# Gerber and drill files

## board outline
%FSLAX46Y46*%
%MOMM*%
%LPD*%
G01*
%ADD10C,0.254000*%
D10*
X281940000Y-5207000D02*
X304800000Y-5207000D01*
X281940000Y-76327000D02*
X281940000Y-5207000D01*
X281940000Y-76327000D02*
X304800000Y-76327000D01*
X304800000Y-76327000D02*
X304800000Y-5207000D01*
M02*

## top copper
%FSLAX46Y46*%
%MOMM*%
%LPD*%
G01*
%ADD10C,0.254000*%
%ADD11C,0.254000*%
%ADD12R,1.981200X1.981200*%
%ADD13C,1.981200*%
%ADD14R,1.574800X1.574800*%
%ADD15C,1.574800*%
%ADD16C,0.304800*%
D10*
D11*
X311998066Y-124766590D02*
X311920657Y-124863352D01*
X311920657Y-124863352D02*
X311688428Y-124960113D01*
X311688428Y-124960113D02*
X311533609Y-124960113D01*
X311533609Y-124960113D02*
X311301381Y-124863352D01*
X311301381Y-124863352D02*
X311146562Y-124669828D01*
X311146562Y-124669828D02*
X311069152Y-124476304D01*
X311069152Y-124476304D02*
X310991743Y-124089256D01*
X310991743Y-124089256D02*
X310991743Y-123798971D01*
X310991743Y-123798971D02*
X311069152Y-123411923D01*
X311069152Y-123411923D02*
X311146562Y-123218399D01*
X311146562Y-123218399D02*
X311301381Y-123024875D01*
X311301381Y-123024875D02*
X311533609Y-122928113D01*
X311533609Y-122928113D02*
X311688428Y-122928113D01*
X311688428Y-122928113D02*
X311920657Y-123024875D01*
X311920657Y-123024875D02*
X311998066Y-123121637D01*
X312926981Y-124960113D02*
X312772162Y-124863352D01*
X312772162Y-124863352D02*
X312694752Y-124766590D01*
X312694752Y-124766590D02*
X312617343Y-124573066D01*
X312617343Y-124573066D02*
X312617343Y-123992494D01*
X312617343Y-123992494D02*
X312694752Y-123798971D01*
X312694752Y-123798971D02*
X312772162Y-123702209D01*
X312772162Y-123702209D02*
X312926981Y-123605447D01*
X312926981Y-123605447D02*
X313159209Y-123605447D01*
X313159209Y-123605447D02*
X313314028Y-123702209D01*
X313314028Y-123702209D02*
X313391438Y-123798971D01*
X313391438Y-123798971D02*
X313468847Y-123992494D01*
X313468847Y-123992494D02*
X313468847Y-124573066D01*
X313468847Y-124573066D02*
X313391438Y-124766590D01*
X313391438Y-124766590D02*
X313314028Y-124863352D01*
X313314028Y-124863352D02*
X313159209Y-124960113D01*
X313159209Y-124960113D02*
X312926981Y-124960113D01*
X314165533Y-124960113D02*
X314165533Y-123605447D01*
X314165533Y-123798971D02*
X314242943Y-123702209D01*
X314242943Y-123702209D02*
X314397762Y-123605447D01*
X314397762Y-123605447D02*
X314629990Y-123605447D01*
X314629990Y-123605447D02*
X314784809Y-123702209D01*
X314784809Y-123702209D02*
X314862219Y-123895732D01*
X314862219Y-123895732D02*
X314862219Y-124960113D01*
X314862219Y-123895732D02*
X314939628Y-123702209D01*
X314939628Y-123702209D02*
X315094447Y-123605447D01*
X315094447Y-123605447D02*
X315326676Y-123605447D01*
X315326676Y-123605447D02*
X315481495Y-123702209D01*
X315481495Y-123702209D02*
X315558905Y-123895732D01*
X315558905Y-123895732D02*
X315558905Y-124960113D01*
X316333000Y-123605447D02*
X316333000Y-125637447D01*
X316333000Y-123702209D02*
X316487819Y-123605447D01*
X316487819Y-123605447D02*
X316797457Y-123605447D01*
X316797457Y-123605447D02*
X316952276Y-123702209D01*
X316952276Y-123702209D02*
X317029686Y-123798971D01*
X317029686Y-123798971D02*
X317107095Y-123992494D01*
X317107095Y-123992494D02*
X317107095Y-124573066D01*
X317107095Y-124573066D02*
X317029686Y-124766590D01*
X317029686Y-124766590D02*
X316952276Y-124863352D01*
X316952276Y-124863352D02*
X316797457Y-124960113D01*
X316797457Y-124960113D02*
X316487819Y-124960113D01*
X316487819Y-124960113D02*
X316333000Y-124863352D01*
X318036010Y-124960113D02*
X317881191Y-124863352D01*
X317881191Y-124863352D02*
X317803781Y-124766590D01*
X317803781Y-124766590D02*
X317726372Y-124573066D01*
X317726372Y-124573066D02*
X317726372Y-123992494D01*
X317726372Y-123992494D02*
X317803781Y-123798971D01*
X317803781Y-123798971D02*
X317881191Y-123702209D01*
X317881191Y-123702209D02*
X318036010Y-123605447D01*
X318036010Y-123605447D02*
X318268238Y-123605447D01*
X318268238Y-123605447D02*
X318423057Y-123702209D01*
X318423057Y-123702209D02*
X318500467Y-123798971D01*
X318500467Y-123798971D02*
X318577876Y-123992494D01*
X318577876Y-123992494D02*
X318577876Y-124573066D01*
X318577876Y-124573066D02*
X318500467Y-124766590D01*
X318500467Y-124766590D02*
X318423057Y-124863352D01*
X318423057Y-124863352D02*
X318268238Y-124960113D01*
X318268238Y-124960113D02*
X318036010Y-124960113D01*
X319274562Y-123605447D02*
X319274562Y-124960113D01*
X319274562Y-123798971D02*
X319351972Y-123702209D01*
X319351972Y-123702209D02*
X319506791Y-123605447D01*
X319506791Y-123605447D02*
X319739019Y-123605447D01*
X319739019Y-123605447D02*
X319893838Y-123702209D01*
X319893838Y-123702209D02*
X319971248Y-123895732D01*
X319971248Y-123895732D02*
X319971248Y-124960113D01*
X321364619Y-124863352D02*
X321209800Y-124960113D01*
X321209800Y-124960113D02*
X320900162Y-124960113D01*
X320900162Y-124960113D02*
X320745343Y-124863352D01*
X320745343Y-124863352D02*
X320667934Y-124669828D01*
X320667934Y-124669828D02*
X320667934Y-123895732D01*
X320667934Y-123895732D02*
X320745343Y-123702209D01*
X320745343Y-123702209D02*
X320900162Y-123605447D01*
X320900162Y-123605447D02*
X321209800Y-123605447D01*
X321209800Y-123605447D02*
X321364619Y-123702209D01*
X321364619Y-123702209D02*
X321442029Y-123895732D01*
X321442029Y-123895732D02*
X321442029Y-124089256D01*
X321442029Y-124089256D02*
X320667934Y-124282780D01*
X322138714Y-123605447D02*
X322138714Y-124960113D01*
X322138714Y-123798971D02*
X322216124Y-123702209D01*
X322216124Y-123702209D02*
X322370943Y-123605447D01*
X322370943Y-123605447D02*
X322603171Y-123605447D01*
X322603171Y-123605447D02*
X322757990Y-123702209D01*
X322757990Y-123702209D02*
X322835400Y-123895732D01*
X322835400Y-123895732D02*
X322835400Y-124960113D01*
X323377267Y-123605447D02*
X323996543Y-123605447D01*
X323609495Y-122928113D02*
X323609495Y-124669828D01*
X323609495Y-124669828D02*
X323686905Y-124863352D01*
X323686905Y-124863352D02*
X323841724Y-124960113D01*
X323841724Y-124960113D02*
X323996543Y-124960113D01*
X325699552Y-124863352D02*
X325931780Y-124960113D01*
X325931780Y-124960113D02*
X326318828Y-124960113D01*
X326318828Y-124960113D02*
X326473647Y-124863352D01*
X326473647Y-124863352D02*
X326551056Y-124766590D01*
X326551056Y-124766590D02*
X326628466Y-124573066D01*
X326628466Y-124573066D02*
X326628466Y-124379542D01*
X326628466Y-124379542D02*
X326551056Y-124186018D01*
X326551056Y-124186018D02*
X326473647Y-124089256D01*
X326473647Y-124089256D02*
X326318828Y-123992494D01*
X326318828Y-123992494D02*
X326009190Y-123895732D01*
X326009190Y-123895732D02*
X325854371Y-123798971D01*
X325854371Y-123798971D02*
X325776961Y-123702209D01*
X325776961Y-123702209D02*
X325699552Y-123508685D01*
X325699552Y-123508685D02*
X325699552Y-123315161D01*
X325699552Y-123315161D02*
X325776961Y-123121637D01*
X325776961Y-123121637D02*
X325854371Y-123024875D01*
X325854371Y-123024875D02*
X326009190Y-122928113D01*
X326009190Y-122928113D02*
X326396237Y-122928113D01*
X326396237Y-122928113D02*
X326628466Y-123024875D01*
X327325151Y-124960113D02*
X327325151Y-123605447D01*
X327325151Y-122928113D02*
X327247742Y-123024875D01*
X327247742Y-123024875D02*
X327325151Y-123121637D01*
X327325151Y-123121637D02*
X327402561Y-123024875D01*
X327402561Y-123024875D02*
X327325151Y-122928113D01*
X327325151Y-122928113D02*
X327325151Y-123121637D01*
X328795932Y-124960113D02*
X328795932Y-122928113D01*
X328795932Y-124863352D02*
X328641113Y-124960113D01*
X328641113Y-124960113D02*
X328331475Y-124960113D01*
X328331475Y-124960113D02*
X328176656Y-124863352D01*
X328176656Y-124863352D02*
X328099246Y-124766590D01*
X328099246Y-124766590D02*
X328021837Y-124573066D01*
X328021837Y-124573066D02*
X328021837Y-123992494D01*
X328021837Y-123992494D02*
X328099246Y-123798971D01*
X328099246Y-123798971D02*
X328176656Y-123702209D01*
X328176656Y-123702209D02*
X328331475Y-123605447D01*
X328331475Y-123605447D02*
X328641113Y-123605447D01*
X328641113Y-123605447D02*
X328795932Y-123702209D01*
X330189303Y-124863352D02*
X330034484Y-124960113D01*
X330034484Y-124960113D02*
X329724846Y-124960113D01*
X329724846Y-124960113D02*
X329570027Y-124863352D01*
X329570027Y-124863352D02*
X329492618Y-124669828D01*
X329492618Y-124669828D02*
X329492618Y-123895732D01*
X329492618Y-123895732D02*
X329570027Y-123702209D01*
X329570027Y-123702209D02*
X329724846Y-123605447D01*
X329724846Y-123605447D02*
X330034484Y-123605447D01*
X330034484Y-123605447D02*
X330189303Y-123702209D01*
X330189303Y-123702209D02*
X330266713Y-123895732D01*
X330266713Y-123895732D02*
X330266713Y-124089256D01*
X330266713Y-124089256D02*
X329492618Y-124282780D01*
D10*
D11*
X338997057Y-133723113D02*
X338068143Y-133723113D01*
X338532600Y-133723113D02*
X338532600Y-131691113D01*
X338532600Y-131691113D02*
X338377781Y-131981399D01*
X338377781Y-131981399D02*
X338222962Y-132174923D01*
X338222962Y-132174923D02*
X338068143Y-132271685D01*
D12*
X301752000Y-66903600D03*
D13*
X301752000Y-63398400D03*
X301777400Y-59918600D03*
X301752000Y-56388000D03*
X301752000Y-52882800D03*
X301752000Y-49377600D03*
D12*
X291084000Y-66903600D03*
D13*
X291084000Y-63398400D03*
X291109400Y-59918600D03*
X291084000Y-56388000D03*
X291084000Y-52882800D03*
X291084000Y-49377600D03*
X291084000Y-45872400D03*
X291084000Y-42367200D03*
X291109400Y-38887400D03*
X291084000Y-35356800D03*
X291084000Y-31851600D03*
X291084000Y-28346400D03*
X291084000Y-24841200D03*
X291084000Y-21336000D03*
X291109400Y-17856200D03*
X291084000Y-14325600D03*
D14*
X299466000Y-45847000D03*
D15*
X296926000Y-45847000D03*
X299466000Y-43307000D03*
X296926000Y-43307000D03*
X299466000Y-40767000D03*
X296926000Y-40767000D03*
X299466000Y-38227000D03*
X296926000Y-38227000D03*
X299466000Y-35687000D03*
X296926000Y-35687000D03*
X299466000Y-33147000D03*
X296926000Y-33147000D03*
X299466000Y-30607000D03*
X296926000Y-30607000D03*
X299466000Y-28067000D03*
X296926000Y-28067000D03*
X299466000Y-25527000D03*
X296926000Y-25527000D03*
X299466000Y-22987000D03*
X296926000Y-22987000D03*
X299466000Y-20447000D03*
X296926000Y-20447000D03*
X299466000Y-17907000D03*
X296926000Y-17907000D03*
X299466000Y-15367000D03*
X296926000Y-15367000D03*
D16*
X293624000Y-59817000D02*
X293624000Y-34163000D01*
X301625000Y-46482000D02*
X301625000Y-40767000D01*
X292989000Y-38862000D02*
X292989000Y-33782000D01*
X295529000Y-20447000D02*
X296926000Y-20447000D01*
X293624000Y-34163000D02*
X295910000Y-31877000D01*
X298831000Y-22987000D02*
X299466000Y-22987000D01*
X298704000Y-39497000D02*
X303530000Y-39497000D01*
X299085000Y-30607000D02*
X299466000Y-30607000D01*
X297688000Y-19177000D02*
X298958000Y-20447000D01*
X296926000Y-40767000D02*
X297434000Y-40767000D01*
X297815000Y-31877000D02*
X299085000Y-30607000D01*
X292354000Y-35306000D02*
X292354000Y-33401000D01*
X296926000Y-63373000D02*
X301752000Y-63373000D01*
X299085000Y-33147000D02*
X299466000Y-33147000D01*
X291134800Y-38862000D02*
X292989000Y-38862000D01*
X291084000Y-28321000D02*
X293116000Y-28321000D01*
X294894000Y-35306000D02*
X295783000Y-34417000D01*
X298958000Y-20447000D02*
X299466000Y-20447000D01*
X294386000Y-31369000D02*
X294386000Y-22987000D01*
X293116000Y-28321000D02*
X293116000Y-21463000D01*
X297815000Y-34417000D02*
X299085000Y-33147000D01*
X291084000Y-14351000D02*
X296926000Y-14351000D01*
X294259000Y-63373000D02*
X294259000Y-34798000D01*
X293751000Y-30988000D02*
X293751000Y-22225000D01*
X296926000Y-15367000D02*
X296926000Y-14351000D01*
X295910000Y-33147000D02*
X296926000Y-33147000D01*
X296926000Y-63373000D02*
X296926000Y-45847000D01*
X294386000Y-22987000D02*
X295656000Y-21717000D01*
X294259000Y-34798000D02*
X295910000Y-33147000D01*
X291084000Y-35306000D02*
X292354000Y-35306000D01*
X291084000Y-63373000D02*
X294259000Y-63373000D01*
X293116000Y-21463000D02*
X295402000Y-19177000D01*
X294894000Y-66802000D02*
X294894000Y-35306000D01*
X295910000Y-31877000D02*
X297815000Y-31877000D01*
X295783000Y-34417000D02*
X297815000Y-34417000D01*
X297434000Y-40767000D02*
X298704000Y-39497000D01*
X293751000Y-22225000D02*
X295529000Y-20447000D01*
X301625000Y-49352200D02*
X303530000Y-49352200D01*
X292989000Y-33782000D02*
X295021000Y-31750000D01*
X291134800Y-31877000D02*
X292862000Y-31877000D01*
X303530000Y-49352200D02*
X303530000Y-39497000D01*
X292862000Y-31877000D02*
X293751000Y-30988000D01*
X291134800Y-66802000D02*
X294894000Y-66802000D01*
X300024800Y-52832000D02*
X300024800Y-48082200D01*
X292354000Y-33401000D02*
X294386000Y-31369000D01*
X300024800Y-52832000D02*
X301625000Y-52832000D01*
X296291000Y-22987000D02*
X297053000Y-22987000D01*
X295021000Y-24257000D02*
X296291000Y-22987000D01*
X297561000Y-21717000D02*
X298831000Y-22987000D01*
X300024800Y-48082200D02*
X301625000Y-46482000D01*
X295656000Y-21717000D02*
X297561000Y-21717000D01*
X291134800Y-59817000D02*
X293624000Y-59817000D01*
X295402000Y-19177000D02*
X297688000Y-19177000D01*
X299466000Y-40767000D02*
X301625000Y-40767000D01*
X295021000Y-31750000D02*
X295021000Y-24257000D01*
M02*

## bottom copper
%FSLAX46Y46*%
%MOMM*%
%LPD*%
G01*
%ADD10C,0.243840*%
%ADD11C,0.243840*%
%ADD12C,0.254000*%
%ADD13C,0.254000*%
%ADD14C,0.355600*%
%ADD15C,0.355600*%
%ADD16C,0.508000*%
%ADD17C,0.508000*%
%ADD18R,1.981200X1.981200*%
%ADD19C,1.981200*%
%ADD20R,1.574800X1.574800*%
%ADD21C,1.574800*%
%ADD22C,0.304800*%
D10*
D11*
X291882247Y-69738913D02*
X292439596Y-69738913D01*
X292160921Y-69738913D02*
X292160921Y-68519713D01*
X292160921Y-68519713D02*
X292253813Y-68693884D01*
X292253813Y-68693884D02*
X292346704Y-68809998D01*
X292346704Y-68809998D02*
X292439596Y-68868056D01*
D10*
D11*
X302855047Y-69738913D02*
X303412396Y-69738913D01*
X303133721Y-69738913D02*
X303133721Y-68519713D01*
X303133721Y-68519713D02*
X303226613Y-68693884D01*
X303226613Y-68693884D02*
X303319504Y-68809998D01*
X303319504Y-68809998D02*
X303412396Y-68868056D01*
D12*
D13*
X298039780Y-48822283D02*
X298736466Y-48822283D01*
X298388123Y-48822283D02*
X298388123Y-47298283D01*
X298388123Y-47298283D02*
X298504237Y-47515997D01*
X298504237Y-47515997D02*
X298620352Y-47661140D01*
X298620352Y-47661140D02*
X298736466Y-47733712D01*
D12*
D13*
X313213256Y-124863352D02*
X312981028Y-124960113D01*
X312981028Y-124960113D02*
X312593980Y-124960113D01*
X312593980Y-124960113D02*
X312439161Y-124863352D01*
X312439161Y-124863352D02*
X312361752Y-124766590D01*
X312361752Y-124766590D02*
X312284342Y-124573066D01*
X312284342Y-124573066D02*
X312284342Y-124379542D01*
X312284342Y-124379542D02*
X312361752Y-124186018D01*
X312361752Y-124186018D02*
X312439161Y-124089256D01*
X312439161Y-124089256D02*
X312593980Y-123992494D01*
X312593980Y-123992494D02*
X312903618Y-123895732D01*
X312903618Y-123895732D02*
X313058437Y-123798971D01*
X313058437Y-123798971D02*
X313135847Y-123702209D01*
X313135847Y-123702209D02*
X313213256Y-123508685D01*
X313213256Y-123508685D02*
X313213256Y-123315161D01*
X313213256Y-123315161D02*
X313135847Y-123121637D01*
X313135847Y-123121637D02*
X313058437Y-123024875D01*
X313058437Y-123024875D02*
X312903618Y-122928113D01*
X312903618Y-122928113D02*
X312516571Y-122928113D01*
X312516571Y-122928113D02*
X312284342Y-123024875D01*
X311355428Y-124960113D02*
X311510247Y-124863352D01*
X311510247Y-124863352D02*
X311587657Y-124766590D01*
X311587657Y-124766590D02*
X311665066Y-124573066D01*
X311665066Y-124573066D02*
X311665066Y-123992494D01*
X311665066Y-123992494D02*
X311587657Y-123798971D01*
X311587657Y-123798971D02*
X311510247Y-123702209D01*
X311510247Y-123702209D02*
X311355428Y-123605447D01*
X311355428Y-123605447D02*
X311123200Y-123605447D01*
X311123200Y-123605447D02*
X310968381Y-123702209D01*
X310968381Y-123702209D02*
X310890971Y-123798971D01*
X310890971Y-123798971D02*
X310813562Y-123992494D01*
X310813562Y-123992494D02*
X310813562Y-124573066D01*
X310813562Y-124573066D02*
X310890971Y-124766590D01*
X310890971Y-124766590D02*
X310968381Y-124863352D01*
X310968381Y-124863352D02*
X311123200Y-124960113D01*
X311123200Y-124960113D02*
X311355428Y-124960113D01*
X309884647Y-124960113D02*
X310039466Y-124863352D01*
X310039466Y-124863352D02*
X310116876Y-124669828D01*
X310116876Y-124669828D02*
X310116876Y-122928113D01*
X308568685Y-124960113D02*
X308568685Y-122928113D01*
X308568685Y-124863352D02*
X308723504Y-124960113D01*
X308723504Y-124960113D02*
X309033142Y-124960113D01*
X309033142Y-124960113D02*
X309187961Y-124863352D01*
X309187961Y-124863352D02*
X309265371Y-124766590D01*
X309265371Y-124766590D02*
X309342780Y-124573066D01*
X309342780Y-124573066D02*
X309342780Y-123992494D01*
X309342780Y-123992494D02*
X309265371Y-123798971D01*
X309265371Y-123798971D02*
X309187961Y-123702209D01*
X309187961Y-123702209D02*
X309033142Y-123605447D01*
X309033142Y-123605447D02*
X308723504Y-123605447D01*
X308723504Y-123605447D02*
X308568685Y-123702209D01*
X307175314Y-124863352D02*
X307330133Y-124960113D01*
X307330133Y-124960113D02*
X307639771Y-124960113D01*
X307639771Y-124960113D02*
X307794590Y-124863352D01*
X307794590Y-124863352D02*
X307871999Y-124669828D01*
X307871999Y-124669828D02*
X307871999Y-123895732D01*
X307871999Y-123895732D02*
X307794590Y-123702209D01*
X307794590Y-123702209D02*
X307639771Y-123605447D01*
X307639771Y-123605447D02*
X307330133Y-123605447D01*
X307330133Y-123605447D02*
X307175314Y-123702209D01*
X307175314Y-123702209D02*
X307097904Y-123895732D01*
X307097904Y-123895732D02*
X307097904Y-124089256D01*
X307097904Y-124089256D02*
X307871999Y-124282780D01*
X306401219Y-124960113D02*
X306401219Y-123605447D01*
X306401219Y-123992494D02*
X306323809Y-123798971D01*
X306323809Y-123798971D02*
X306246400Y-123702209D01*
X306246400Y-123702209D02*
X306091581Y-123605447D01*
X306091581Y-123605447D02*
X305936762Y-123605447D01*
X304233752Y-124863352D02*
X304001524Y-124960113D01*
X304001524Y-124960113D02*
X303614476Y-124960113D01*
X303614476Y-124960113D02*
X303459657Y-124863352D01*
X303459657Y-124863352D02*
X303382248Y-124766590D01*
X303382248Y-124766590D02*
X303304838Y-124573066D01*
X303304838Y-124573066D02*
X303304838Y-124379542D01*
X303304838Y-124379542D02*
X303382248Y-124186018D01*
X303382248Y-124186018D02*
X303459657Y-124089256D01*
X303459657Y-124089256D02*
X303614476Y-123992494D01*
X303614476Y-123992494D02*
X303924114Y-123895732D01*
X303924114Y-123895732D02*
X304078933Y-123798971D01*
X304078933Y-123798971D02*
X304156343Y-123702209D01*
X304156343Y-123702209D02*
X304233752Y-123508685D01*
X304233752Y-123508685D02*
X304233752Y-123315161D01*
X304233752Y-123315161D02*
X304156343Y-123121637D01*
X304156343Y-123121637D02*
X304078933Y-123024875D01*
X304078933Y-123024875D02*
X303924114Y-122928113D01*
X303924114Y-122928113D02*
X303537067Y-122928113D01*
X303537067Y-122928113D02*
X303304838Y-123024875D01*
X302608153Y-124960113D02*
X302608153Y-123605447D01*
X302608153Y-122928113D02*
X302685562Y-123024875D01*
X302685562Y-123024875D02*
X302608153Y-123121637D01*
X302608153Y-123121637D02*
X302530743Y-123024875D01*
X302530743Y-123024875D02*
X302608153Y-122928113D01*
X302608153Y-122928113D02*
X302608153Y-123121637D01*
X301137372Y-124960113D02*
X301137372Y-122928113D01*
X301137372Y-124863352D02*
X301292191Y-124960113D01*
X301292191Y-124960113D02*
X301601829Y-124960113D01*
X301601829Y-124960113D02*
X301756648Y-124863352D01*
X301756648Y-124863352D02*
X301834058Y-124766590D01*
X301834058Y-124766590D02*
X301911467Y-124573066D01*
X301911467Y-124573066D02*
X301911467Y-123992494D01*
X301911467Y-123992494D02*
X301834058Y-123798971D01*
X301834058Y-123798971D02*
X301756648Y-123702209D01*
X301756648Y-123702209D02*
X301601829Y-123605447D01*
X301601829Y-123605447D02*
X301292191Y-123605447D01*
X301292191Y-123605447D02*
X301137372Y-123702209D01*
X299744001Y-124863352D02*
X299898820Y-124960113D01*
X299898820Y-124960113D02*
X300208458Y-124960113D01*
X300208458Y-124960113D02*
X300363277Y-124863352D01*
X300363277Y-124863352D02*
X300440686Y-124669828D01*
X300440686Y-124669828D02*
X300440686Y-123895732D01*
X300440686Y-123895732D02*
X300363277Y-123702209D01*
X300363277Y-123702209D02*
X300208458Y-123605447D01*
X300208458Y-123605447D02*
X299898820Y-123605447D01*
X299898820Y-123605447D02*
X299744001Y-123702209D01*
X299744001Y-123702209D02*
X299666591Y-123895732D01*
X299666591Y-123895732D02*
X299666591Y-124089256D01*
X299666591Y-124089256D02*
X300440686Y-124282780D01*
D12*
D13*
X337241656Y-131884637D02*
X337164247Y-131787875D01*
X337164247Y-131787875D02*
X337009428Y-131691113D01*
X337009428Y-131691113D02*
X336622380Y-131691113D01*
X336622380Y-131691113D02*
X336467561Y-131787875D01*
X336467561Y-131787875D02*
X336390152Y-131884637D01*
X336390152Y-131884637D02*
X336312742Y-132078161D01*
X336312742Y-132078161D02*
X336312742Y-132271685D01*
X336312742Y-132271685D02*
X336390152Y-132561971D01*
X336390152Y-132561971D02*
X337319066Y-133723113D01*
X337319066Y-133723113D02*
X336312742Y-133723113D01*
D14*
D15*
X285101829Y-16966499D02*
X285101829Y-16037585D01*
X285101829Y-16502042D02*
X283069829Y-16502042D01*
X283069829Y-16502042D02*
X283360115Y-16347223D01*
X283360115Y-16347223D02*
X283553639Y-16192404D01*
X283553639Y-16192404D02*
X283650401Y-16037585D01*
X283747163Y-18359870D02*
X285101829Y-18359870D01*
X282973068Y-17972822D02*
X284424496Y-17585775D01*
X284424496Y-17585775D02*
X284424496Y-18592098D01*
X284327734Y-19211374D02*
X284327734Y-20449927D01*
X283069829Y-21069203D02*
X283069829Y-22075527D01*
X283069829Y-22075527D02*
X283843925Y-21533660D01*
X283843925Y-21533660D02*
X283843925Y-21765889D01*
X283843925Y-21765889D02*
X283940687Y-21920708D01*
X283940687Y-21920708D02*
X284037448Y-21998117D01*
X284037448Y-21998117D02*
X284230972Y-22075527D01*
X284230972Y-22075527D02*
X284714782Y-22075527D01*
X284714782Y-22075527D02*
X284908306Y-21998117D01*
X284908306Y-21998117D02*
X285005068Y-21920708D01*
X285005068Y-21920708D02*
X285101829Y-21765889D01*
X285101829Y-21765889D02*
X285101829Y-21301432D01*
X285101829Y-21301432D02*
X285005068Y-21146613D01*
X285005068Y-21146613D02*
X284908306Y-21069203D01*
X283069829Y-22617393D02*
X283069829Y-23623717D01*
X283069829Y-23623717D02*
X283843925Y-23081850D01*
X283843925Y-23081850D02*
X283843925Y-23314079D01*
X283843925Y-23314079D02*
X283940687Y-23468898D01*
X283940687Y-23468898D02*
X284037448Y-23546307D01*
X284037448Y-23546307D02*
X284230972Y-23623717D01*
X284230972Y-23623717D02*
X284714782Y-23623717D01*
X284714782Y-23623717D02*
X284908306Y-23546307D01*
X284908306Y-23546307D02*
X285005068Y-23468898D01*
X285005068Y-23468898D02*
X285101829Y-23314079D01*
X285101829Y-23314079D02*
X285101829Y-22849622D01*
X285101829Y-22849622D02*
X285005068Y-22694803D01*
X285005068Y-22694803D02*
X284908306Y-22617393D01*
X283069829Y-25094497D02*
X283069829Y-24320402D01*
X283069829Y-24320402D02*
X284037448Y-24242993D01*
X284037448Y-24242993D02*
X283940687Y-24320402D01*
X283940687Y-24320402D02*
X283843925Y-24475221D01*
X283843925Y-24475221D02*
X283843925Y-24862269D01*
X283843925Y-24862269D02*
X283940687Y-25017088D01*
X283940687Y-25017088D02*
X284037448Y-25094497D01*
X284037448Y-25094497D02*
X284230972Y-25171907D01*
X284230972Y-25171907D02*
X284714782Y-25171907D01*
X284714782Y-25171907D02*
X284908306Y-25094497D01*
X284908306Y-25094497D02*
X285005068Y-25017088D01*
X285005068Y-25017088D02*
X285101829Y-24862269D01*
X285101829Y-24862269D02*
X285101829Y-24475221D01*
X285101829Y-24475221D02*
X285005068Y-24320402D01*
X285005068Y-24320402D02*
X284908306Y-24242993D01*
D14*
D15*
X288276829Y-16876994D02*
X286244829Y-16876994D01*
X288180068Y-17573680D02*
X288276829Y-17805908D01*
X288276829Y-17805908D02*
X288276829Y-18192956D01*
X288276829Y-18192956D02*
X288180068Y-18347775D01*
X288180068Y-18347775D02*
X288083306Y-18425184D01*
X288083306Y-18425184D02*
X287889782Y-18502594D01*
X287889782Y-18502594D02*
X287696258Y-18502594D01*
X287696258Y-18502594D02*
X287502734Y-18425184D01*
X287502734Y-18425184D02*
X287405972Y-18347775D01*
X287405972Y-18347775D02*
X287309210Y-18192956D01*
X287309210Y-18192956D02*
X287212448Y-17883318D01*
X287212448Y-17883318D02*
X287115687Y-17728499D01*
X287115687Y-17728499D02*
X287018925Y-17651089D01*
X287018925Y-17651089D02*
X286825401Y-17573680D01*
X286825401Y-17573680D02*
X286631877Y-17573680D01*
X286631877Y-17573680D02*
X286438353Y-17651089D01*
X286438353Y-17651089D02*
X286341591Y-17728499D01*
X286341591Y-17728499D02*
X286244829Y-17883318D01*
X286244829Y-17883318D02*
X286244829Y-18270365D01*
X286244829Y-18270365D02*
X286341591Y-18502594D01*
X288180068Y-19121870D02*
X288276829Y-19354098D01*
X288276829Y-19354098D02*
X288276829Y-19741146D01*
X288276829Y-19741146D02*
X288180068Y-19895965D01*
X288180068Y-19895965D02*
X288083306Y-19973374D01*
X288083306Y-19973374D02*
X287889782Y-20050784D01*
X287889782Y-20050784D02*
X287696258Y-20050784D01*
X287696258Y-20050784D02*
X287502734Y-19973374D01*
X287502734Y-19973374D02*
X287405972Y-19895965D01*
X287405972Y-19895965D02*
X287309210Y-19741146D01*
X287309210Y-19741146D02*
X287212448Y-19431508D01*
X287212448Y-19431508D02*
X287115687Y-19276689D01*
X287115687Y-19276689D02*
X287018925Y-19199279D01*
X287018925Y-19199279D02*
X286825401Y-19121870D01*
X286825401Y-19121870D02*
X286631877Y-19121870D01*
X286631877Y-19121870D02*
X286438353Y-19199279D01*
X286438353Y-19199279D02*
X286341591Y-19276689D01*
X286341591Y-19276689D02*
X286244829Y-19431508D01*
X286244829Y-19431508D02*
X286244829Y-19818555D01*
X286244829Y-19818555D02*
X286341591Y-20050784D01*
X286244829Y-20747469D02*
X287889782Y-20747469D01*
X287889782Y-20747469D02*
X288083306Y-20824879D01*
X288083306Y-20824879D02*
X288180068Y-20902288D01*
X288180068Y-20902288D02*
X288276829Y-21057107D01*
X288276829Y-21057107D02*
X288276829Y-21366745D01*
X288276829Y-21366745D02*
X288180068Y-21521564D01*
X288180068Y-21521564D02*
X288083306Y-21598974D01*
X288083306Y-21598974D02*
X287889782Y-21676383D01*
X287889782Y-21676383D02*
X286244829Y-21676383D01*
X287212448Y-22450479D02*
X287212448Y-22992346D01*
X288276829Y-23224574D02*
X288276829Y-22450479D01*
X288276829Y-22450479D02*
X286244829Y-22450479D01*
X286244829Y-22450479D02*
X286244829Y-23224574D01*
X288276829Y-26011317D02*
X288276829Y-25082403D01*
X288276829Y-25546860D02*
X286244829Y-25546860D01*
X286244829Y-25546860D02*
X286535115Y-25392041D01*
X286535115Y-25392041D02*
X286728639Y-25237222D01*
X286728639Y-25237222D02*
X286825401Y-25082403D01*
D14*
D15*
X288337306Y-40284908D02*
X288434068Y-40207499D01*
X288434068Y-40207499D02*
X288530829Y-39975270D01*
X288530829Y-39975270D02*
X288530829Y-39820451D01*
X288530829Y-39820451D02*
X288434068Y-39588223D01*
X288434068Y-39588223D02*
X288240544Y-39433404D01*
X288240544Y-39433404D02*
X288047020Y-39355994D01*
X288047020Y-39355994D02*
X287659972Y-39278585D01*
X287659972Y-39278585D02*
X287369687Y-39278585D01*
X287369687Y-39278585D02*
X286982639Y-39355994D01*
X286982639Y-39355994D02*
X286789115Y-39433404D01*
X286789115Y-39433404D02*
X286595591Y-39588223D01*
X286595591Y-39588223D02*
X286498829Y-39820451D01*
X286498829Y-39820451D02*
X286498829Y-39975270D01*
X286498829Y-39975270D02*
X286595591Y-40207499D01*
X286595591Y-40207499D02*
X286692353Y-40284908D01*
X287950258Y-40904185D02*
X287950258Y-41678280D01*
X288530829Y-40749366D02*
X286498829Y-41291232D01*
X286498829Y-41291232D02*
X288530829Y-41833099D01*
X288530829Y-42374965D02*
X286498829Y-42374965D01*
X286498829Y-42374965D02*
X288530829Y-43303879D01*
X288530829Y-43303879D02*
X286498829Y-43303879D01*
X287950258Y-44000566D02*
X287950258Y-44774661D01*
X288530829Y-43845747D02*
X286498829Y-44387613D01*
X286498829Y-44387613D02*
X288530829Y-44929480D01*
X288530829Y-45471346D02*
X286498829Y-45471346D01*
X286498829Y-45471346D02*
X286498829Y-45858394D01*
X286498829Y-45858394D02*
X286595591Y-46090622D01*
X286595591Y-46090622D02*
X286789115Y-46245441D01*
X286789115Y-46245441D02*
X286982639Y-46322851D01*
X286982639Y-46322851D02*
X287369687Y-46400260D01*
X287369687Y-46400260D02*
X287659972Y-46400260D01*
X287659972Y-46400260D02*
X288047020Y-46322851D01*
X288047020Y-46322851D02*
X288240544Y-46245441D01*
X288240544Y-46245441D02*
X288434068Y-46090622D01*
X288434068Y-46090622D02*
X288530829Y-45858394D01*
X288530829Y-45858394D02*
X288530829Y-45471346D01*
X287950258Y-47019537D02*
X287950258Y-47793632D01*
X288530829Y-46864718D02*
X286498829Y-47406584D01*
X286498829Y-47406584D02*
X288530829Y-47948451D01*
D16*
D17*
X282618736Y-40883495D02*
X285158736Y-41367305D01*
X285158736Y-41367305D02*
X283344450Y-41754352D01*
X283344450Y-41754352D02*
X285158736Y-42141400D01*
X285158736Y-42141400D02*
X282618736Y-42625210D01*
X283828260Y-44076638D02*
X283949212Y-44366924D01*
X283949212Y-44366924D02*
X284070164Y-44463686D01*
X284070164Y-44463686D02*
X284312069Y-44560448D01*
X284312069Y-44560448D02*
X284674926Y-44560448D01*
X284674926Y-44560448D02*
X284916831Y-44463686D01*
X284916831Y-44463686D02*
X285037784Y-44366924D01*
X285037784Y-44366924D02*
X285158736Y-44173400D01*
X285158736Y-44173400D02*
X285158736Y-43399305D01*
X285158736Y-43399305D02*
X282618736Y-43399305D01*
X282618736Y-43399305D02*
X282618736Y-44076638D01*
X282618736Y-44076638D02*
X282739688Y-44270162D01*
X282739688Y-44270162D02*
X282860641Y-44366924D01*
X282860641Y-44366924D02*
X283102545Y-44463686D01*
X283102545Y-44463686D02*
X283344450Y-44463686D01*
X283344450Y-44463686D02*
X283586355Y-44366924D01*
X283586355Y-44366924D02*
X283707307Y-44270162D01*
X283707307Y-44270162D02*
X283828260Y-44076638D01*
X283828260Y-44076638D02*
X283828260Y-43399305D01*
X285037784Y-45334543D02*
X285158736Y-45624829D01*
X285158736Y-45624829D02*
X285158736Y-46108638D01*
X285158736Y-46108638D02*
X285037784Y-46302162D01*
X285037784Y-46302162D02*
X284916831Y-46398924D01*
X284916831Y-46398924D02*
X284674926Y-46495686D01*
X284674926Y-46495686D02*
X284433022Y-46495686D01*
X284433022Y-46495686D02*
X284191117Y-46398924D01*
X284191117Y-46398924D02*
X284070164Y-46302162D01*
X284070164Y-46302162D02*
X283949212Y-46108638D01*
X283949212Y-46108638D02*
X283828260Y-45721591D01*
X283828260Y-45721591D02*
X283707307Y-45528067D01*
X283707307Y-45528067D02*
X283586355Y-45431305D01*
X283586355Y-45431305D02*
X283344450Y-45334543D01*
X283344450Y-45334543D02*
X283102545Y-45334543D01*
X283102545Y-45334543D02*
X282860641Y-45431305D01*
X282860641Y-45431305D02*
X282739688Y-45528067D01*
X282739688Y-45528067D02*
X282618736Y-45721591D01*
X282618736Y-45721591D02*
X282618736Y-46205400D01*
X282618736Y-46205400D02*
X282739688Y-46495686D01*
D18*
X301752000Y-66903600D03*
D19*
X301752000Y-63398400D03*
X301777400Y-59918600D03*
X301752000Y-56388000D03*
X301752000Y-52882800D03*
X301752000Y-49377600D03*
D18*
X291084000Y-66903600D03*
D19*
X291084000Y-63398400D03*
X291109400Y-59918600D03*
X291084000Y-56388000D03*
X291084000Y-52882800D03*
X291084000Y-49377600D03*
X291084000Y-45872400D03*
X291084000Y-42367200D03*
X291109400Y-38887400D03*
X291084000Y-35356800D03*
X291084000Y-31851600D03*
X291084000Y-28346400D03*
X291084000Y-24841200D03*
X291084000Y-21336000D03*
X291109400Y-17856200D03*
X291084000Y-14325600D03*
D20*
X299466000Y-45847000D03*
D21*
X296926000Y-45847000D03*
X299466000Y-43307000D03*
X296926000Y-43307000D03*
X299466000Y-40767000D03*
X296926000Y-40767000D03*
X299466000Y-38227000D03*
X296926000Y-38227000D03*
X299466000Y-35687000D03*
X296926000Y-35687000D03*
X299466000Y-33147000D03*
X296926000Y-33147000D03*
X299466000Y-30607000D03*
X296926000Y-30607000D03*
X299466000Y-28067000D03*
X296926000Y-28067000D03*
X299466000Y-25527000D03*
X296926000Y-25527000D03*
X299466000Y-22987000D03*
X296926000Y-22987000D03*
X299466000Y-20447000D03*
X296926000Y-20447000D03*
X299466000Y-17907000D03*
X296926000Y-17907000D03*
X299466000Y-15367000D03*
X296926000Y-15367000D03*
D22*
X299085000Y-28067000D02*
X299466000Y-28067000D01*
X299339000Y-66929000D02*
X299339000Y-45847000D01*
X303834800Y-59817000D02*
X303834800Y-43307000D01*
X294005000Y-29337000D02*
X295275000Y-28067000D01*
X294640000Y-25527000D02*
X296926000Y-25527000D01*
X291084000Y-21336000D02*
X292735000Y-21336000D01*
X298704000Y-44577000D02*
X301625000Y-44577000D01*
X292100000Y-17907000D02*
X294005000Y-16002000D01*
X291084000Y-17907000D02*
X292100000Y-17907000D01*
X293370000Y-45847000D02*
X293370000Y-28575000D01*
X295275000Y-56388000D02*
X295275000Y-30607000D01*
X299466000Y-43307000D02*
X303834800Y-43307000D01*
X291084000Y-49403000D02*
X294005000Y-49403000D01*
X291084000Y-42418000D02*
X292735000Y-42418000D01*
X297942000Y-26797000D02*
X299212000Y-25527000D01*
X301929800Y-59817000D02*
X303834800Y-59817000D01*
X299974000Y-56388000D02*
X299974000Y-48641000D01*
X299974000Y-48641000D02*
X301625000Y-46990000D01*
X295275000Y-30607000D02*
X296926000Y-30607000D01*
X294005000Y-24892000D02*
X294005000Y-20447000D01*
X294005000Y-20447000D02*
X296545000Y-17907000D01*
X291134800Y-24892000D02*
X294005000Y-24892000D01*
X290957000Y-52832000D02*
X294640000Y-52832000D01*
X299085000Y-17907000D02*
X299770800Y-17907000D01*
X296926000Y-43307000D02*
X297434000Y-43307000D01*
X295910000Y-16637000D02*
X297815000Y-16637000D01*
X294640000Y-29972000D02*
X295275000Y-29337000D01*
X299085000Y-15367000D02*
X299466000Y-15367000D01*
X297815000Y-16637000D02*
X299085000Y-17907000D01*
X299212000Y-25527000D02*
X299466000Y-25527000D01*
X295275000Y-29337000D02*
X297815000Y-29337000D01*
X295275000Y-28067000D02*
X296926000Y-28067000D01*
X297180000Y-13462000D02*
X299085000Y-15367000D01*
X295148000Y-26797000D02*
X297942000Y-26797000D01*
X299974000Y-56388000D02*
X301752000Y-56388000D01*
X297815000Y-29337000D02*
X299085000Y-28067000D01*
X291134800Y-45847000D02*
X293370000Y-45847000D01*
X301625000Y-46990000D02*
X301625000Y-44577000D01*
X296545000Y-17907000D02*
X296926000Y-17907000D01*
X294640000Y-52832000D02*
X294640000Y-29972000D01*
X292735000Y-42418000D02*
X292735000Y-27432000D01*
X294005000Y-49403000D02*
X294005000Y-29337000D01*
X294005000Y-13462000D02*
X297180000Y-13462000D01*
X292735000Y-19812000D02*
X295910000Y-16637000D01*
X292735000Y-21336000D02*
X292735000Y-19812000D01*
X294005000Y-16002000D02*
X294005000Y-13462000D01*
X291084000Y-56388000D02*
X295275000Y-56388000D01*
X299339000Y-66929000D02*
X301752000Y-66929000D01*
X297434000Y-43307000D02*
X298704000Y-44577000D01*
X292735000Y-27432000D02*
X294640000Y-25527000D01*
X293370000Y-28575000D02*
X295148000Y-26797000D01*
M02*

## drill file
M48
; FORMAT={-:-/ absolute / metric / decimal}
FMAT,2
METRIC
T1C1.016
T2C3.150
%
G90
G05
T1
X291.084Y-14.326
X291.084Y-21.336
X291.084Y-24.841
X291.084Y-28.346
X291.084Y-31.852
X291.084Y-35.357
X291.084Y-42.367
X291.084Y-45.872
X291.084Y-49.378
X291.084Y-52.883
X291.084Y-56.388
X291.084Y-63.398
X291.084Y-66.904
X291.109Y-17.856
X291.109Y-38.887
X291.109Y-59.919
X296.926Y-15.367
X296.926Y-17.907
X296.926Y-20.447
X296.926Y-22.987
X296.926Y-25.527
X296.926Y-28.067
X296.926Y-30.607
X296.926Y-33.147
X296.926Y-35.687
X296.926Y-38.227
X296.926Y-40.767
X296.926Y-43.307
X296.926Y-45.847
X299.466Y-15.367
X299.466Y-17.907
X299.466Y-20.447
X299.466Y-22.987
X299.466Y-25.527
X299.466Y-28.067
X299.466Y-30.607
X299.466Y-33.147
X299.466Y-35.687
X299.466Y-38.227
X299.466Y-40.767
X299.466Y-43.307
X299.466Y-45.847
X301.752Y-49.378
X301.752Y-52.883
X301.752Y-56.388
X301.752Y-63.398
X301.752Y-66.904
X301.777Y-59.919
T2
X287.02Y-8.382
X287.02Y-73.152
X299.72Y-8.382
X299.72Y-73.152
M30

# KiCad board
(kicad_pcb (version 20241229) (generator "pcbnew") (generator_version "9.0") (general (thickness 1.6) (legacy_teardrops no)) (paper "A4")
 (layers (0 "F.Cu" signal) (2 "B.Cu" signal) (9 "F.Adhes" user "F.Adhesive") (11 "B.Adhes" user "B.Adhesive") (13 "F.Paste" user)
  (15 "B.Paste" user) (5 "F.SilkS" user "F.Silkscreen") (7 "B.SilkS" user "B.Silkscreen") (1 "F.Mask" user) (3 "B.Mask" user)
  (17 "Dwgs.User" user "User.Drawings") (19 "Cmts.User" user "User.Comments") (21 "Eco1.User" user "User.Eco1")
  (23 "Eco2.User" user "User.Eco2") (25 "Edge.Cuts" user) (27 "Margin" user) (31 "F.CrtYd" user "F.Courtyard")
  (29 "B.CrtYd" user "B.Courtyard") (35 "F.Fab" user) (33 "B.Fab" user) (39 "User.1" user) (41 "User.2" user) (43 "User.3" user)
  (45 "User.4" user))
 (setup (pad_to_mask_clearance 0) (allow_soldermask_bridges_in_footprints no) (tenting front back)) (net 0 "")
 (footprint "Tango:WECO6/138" (layer "F.Cu") (at 301.752 66.9036)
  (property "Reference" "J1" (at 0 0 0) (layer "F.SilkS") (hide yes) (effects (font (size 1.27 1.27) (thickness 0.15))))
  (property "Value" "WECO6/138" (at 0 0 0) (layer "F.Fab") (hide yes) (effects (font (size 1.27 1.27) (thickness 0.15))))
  (pad "1" thru_hole rect (at 0 0) (size 1.9812 1.9812) (drill 1.016) (layers "*.Cu" "*.Mask") (remove_unused_layers no)
   (thermal_bridge_angle 45))
  (pad "2" thru_hole circle (at 0 -3.5052) (size 1.9812 1.9812) (drill 1.016) (layers "*.Cu" "*.Mask") (remove_unused_layers no))
  (pad "3" thru_hole circle (at 0.0254 -6.985) (size 1.9812 1.9812) (drill 1.016) (layers "*.Cu" "*.Mask") (remove_unused_layers no))
  (pad "4" thru_hole circle (at 0 -10.5156) (size 1.9812 1.9812) (drill 1.016) (layers "*.Cu" "*.Mask") (remove_unused_layers no))
  (pad "5" thru_hole circle (at 0 -14.0208) (size 1.9812 1.9812) (drill 1.016) (layers "*.Cu" "*.Mask") (remove_unused_layers no))
  (pad "6" thru_hole circle (at 0 -17.526) (size 1.9812 1.9812) (drill 1.016) (layers "*.Cu" "*.Mask") (remove_unused_layers no)))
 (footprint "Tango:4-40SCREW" (layer "F.Cu") (at 299.72 73.152)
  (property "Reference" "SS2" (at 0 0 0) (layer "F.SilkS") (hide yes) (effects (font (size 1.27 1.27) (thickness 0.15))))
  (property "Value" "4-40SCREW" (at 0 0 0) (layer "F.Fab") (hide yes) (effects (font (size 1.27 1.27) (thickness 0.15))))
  (pad "" np_thru_hole circle (at 0 0) (size 3.1496 3.1496) (drill 3.1496) (layers "*.Cu" "*.Mask")))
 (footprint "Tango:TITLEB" (layer "F.Cu") (at 358.14 139.827)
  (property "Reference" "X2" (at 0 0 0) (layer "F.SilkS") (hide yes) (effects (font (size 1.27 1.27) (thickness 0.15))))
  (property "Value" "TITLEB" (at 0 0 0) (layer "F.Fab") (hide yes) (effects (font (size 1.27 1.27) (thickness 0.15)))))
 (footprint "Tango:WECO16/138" (layer "F.Cu") (at 291.084 66.9036)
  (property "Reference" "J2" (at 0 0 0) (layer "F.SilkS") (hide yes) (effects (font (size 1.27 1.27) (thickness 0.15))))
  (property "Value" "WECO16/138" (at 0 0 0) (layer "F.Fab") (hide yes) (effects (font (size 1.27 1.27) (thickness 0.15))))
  (pad "1" thru_hole rect (at 0 0) (size 1.9812 1.9812) (drill 1.016) (layers "*.Cu" "*.Mask") (remove_unused_layers no)
   (thermal_bridge_angle 45))
  (pad "2" thru_hole circle (at 0 -3.5052) (size 1.9812 1.9812) (drill 1.016) (layers "*.Cu" "*.Mask") (remove_unused_layers no))
  (pad "3" thru_hole circle (at 0.0254 -6.985) (size 1.9812 1.9812) (drill 1.016) (layers "*.Cu" "*.Mask") (remove_unused_layers no))
  (pad "4" thru_hole circle (at 0 -10.5156) (size 1.9812 1.9812) (drill 1.016) (layers "*.Cu" "*.Mask") (remove_unused_layers no))
  (pad "5" thru_hole circle (at 0 -14.0208) (size 1.9812 1.9812) (drill 1.016) (layers "*.Cu" "*.Mask") (remove_unused_layers no))
  (pad "6" thru_hole circle (at 0 -17.526) (size 1.9812 1.9812) (drill 1.016) (layers "*.Cu" "*.Mask") (remove_unused_layers no))
  (pad "7" thru_hole circle (at 0 -21.0312) (size 1.9812 1.9812) (drill 1.016) (layers "*.Cu" "*.Mask") (remove_unused_layers no))
  (pad "8" thru_hole circle (at 0 -24.5364) (size 1.9812 1.9812) (drill 1.016) (layers "*.Cu" "*.Mask") (remove_unused_layers no))
  (pad "9" thru_hole circle (at 0.0254 -28.0162) (size 1.9812 1.9812) (drill 1.016) (layers "*.Cu" "*.Mask") (remove_unused_layers no))
  (pad "10" thru_hole circle (at 0 -31.5468) (size 1.9812 1.9812) (drill 1.016) (layers "*.Cu" "*.Mask") (remove_unused_layers no))
  (pad "11" thru_hole circle (at 0 -35.052) (size 1.9812 1.9812) (drill 1.016) (layers "*.Cu" "*.Mask") (remove_unused_layers no))
  (pad "12" thru_hole circle (at 0 -38.5572) (size 1.9812 1.9812) (drill 1.016) (layers "*.Cu" "*.Mask") (remove_unused_layers no))
  (pad "13" thru_hole circle (at 0 -42.0624) (size 1.9812 1.9812) (drill 1.016) (layers "*.Cu" "*.Mask") (remove_unused_layers no))
  (pad "14" thru_hole circle (at 0 -45.5676) (size 1.9812 1.9812) (drill 1.016) (layers "*.Cu" "*.Mask") (remove_unused_layers no))
  (pad "15" thru_hole circle (at 0.0254 -49.0474) (size 1.9812 1.9812) (drill 1.016) (layers "*.Cu" "*.Mask") (remove_unused_layers no))
  (pad "16" thru_hole circle (at 0 -52.578) (size 1.9812 1.9812) (drill 1.016) (layers "*.Cu" "*.Mask") (remove_unused_layers no)))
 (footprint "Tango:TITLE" (layer "F.Cu") (at 359.41 134.747)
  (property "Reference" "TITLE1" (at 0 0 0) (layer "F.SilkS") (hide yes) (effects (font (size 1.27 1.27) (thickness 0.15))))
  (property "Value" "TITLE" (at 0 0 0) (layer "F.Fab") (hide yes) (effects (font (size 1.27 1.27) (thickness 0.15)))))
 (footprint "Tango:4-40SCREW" (layer "F.Cu") (at 299.72 8.382)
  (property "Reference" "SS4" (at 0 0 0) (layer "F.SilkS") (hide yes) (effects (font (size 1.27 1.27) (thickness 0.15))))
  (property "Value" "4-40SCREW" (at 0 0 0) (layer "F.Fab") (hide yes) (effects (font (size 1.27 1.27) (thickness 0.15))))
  (pad "" np_thru_hole circle (at 0 0) (size 3.1496 3.1496) (drill 3.1496) (layers "*.Cu" "*.Mask")))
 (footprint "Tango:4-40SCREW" (layer "F.Cu") (at 287.02 73.152)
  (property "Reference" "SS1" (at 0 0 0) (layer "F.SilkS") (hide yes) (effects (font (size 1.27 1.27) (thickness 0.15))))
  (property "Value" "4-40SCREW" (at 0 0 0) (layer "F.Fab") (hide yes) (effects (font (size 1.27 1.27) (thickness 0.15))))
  (pad "" np_thru_hole circle (at 0 0) (size 3.1496 3.1496) (drill 3.1496) (layers "*.Cu" "*.Mask")))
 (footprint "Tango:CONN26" (layer "F.Cu") (at 299.466 45.847)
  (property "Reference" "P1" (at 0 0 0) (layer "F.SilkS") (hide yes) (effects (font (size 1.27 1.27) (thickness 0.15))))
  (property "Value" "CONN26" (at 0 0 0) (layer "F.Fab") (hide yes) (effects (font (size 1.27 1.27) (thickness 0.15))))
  (pad "1" thru_hole rect (at 0 0) (size 1.5748 1.5748) (drill 1.016) (layers "*.Cu" "*.Mask") (remove_unused_layers no)
   (thermal_bridge_angle 45))
  (pad "2" thru_hole circle (at -2.54 0) (size 1.5748 1.5748) (drill 1.016) (layers "*.Cu" "*.Mask") (remove_unused_layers no))
  (pad "3" thru_hole circle (at 0 -2.54) (size 1.5748 1.5748) (drill 1.016) (layers "*.Cu" "*.Mask") (remove_unused_layers no))
  (pad "4" thru_hole circle (at -2.54 -2.54) (size 1.5748 1.5748) (drill 1.016) (layers "*.Cu" "*.Mask") (remove_unused_layers no))
  (pad "5" thru_hole circle (at 0 -5.08) (size 1.5748 1.5748) (drill 1.016) (layers "*.Cu" "*.Mask") (remove_unused_layers no))
  (pad "6" thru_hole circle (at -2.54 -5.08) (size 1.5748 1.5748) (drill 1.016) (layers "*.Cu" "*.Mask") (remove_unused_layers no))
  (pad "7" thru_hole circle (at 0 -7.62) (size 1.5748 1.5748) (drill 1.016) (layers "*.Cu" "*.Mask") (remove_unused_layers no))
  (pad "8" thru_hole circle (at -2.54 -7.62) (size 1.5748 1.5748) (drill 1.016) (layers "*.Cu" "*.Mask") (remove_unused_layers no))
  (pad "9" thru_hole circle (at 0 -10.16) (size 1.5748 1.5748) (drill 1.016) (layers "*.Cu" "*.Mask") (remove_unused_layers no))
  (pad "10" thru_hole circle (at -2.54 -10.16) (size 1.5748 1.5748) (drill 1.016) (layers "*.Cu" "*.Mask") (remove_unused_layers no))
  (pad "11" thru_hole circle (at 0 -12.7) (size 1.5748 1.5748) (drill 1.016) (layers "*.Cu" "*.Mask") (remove_unused_layers no))
  (pad "12" thru_hole circle (at -2.54 -12.7) (size 1.5748 1.5748) (drill 1.016) (layers "*.Cu" "*.Mask") (remove_unused_layers no))
  (pad "13" thru_hole circle (at 0 -15.24) (size 1.5748 1.5748) (drill 1.016) (layers "*.Cu" "*.Mask") (remove_unused_layers no))
  (pad "14" thru_hole circle (at -2.54 -15.24) (size 1.5748 1.5748) (drill 1.016) (layers "*.Cu" "*.Mask") (remove_unused_layers no))
  (pad "15" thru_hole circle (at 0 -17.78) (size 1.5748 1.5748) (drill 1.016) (layers "*.Cu" "*.Mask") (remove_unused_layers no))
  (pad "16" thru_hole circle (at -2.54 -17.78) (size 1.5748 1.5748) (drill 1.016) (layers "*.Cu" "*.Mask") (remove_unused_layers no))
  (pad "17" thru_hole circle (at 0 -20.32) (size 1.5748 1.5748) (drill 1.016) (layers "*.Cu" "*.Mask") (remove_unused_layers no))
  (pad "18" thru_hole circle (at -2.54 -20.32) (size 1.5748 1.5748) (drill 1.016) (layers "*.Cu" "*.Mask") (remove_unused_layers no))
  (pad "19" thru_hole circle (at 0 -22.86) (size 1.5748 1.5748) (drill 1.016) (layers "*.Cu" "*.Mask") (remove_unused_layers no))
  (pad "20" thru_hole circle (at -2.54 -22.86) (size 1.5748 1.5748) (drill 1.016) (layers "*.Cu" "*.Mask") (remove_unused_layers no))
  (pad "21" thru_hole circle (at 0 -25.4) (size 1.5748 1.5748) (drill 1.016) (layers "*.Cu" "*.Mask") (remove_unused_layers no))
  (pad "22" thru_hole circle (at -2.54 -25.4) (size 1.5748 1.5748) (drill 1.016) (layers "*.Cu" "*.Mask") (remove_unused_layers no))
  (pad "23" thru_hole circle (at 0 -27.94) (size 1.5748 1.5748) (drill 1.016) (layers "*.Cu" "*.Mask") (remove_unused_layers no))
  (pad "24" thru_hole circle (at -2.54 -27.94) (size 1.5748 1.5748) (drill 1.016) (layers "*.Cu" "*.Mask") (remove_unused_layers no))
  (pad "25" thru_hole circle (at 0 -30.48) (size 1.5748 1.5748) (drill 1.016) (layers "*.Cu" "*.Mask") (remove_unused_layers no))
  (pad "26" thru_hole circle (at -2.54 -30.48) (size 1.5748 1.5748) (drill 1.016) (layers "*.Cu" "*.Mask") (remove_unused_layers no)))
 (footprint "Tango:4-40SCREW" (layer "F.Cu") (at 287.02 8.382)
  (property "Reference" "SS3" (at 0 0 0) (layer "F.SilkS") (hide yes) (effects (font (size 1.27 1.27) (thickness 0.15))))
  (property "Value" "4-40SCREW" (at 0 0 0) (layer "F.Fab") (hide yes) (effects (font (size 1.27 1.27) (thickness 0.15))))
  (pad "" np_thru_hole circle (at 0 0) (size 3.1496 3.1496) (drill 3.1496) (layers "*.Cu" "*.Mask")))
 (gr_line (start 281.94 5.207) (end 304.8 5.207) (stroke (width 0.254) (type default)) (layer "Edge.Cuts"))
 (gr_line (start 281.94 76.327) (end 281.94 5.207) (stroke (width 0.254) (type default)) (layer "Edge.Cuts"))
 (gr_line (start 281.94 76.327) (end 304.8 76.327) (stroke (width 0.254) (type default)) (layer "Edge.Cuts"))
 (gr_line (start 304.8 76.327) (end 304.8 5.207) (stroke (width 0.254) (type default)) (layer "Edge.Cuts"))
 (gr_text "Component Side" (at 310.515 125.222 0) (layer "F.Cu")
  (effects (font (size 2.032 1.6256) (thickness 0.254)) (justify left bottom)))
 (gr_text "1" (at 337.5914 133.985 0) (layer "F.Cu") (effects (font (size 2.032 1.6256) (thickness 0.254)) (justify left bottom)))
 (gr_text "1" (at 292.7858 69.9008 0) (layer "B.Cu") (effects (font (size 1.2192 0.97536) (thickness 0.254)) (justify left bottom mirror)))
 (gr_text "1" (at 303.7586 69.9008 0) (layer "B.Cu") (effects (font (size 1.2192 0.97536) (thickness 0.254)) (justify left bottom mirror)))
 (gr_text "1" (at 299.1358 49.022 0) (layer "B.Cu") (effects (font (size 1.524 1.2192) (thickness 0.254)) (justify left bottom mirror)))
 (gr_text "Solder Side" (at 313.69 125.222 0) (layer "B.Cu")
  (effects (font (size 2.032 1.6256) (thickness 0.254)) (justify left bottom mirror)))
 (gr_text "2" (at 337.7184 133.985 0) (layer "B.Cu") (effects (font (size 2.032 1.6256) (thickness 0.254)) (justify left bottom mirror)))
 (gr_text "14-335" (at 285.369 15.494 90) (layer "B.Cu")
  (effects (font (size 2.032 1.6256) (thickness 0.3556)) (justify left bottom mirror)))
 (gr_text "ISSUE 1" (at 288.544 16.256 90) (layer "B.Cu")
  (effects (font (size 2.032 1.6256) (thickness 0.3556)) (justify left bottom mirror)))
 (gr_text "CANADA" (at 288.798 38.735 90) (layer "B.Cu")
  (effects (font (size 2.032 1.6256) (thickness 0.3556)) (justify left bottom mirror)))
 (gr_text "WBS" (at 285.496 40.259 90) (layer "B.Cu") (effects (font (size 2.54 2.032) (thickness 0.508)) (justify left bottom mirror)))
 (segment (start 293.624 59.817) (end 293.624 34.163) (width 0.3048) (layer "F.Cu") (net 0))
 (segment (start 301.625 46.482) (end 301.625 40.767) (width 0.3048) (layer "F.Cu") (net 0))
 (segment (start 292.989 38.862) (end 292.989 33.782) (width 0.3048) (layer "F.Cu") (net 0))
 (segment (start 295.529 20.447) (end 296.926 20.447) (width 0.3048) (layer "F.Cu") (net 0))
 (segment (start 293.624 34.163) (end 295.91 31.877) (width 0.3048) (layer "F.Cu") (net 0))
 (segment (start 298.831 22.987) (end 299.466 22.987) (width 0.3048) (layer "F.Cu") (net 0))
 (segment (start 298.704 39.497) (end 303.53 39.497) (width 0.3048) (layer "F.Cu") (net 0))
 (segment (start 299.085 30.607) (end 299.466 30.607) (width 0.3048) (layer "F.Cu") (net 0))
 (segment (start 297.688 19.177) (end 298.958 20.447) (width 0.3048) (layer "F.Cu") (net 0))
 (segment (start 296.926 40.767) (end 297.434 40.767) (width 0.3048) (layer "F.Cu") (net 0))
 (segment (start 297.815 31.877) (end 299.085 30.607) (width 0.3048) (layer "F.Cu") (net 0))
 (segment (start 292.354 35.306) (end 292.354 33.401) (width 0.3048) (layer "F.Cu") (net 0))
 (segment (start 296.926 63.373) (end 301.752 63.373) (width 0.3048) (layer "F.Cu") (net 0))
 (segment (start 299.085 33.147) (end 299.466 33.147) (width 0.3048) (layer "F.Cu") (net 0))
 (segment (start 291.1348 38.862) (end 292.989 38.862) (width 0.3048) (layer "F.Cu") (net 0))
 (segment (start 291.084 28.321) (end 293.116 28.321) (width 0.3048) (layer "F.Cu") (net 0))
 (segment (start 294.894 35.306) (end 295.783 34.417) (width 0.3048) (layer "F.Cu") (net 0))
 (segment (start 298.958 20.447) (end 299.466 20.447) (width 0.3048) (layer "F.Cu") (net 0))
 (segment (start 294.386 31.369) (end 294.386 22.987) (width 0.3048) (layer "F.Cu") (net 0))
 (segment (start 293.116 28.321) (end 293.116 21.463) (width 0.3048) (layer "F.Cu") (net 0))
 (segment (start 297.815 34.417) (end 299.085 33.147) (width 0.3048) (layer "F.Cu") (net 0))
 (segment (start 291.084 14.351) (end 296.926 14.351) (width 0.3048) (layer "F.Cu") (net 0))
 (segment (start 294.259 63.373) (end 294.259 34.798) (width 0.3048) (layer "F.Cu") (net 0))
 (segment (start 293.751 30.988) (end 293.751 22.225) (width 0.3048) (layer "F.Cu") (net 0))
 (segment (start 296.926 15.367) (end 296.926 14.351) (width 0.3048) (layer "F.Cu") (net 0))
 (segment (start 295.91 33.147) (end 296.926 33.147) (width 0.3048) (layer "F.Cu") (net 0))
 (segment (start 296.926 63.373) (end 296.926 45.847) (width 0.3048) (layer "F.Cu") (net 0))
 (segment (start 294.386 22.987) (end 295.656 21.717) (width 0.3048) (layer "F.Cu") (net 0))
 (segment (start 294.259 34.798) (end 295.91 33.147) (width 0.3048) (layer "F.Cu") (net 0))
 (segment (start 291.084 35.306) (end 292.354 35.306) (width 0.3048) (layer "F.Cu") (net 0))
 (segment (start 291.084 63.373) (end 294.259 63.373) (width 0.3048) (layer "F.Cu") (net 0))
 (segment (start 293.116 21.463) (end 295.402 19.177) (width 0.3048) (layer "F.Cu") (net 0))
 (segment (start 294.894 66.802) (end 294.894 35.306) (width 0.3048) (layer "F.Cu") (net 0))
 (segment (start 295.91 31.877) (end 297.815 31.877) (width 0.3048) (layer "F.Cu") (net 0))
 (segment (start 295.783 34.417) (end 297.815 34.417) (width 0.3048) (layer "F.Cu") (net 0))
 (segment (start 297.434 40.767) (end 298.704 39.497) (width 0.3048) (layer "F.Cu") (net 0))
 (segment (start 293.751 22.225) (end 295.529 20.447) (width 0.3048) (layer "F.Cu") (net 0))
 (segment (start 301.625 49.3522) (end 303.53 49.3522) (width 0.3048) (layer "F.Cu") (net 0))
 (segment (start 292.989 33.782) (end 295.021 31.75) (width 0.3048) (layer "F.Cu") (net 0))
 (segment (start 291.1348 31.877) (end 292.862 31.877) (width 0.3048) (layer "F.Cu") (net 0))
 (segment (start 303.53 49.3522) (end 303.53 39.497) (width 0.3048) (layer "F.Cu") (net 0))
 (segment (start 292.862 31.877) (end 293.751 30.988) (width 0.3048) (layer "F.Cu") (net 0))
 (segment (start 291.1348 66.802) (end 294.894 66.802) (width 0.3048) (layer "F.Cu") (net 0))
 (segment (start 300.0248 52.832) (end 300.0248 48.0822) (width 0.3048) (layer "F.Cu") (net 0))
 (segment (start 292.354 33.401) (end 294.386 31.369) (width 0.3048) (layer "F.Cu") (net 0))
 (segment (start 300.0248 52.832) (end 301.625 52.832) (width 0.3048) (layer "F.Cu") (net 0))
 (segment (start 296.291 22.987) (end 297.053 22.987) (width 0.3048) (layer "F.Cu") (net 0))
 (segment (start 295.021 24.257) (end 296.291 22.987) (width 0.3048) (layer "F.Cu") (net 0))
 (segment (start 297.561 21.717) (end 298.831 22.987) (width 0.3048) (layer "F.Cu") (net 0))
 (segment (start 300.0248 48.0822) (end 301.625 46.482) (width 0.3048) (layer "F.Cu") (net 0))
 (segment (start 295.656 21.717) (end 297.561 21.717) (width 0.3048) (layer "F.Cu") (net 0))
 (segment (start 291.1348 59.817) (end 293.624 59.817) (width 0.3048) (layer "F.Cu") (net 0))
 (segment (start 295.402 19.177) (end 297.688 19.177) (width 0.3048) (layer "F.Cu") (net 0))
 (segment (start 299.466 40.767) (end 301.625 40.767) (width 0.3048) (layer "F.Cu") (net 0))
 (segment (start 295.021 31.75) (end 295.021 24.257) (width 0.3048) (layer "F.Cu") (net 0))
 (segment (start 299.085 28.067) (end 299.466 28.067) (width 0.3048) (layer "B.Cu") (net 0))
 (segment (start 299.339 66.929) (end 299.339 45.847) (width 0.3048) (layer "B.Cu") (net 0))
 (segment (start 303.8348 59.817) (end 303.8348 43.307) (width 0.3048) (layer "B.Cu") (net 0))
 (segment (start 294.005 29.337) (end 295.275 28.067) (width 0.3048) (layer "B.Cu") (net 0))
 (segment (start 294.64 25.527) (end 296.926 25.527) (width 0.3048) (layer "B.Cu") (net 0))
 (segment (start 291.084 21.336) (end 292.735 21.336) (width 0.3048) (layer "B.Cu") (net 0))
 (segment (start 298.704 44.577) (end 301.625 44.577) (width 0.3048) (layer "B.Cu") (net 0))
 (segment (start 292.1 17.907) (end 294.005 16.002) (width 0.3048) (layer "B.Cu") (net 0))
 (segment (start 291.084 17.907) (end 292.1 17.907) (width 0.3048) (layer "B.Cu") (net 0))
 (segment (start 293.37 45.847) (end 293.37 28.575) (width 0.3048) (layer "B.Cu") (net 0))
 (segment (start 295.275 56.388) (end 295.275 30.607) (width 0.3048) (layer "B.Cu") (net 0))
 (segment (start 299.466 43.307) (end 303.8348 43.307) (width 0.3048) (layer "B.Cu") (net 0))
 (segment (start 291.084 49.403) (end 294.005 49.403) (width 0.3048) (layer "B.Cu") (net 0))
 (segment (start 291.084 42.418) (end 292.735 42.418) (width 0.3048) (layer "B.Cu") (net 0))
 (segment (start 297.942 26.797) (end 299.212 25.527) (width 0.3048) (layer "B.Cu") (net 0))
 (segment (start 301.9298 59.817) (end 303.8348 59.817) (width 0.3048) (layer "B.Cu") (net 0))
 (segment (start 299.974 56.388) (end 299.974 48.641) (width 0.3048) (layer "B.Cu") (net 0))
 (segment (start 299.974 48.641) (end 301.625 46.99) (width 0.3048) (layer "B.Cu") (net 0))
 (segment (start 295.275 30.607) (end 296.926 30.607) (width 0.3048) (layer "B.Cu") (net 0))
 (segment (start 294.005 24.892) (end 294.005 20.447) (width 0.3048) (layer "B.Cu") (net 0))
 (segment (start 294.005 20.447) (end 296.545 17.907) (width 0.3048) (layer "B.Cu") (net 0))
 (segment (start 291.1348 24.892) (end 294.005 24.892) (width 0.3048) (layer "B.Cu") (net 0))
 (segment (start 290.957 52.832) (end 294.64 52.832) (width 0.3048) (layer "B.Cu") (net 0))
 (segment (start 299.085 17.907) (end 299.7708 17.907) (width 0.3048) (layer "B.Cu") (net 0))
 (segment (start 296.926 43.307) (end 297.434 43.307) (width 0.3048) (layer "B.Cu") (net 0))
 (segment (start 295.91 16.637) (end 297.815 16.637) (width 0.3048) (layer "B.Cu") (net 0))
 (segment (start 294.64 29.972) (end 295.275 29.337) (width 0.3048) (layer "B.Cu") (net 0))
 (segment (start 299.085 15.367) (end 299.466 15.367) (width 0.3048) (layer "B.Cu") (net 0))
 (segment (start 297.815 16.637) (end 299.085 17.907) (width 0.3048) (layer "B.Cu") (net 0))
 (segment (start 299.212 25.527) (end 299.466 25.527) (width 0.3048) (layer "B.Cu") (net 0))
 (segment (start 295.275 29.337) (end 297.815 29.337) (width 0.3048) (layer "B.Cu") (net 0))
 (segment (start 295.275 28.067) (end 296.926 28.067) (width 0.3048) (layer "B.Cu") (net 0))
 (segment (start 297.18 13.462) (end 299.085 15.367) (width 0.3048) (layer "B.Cu") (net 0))
 (segment (start 295.148 26.797) (end 297.942 26.797) (width 0.3048) (layer "B.Cu") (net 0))
 (segment (start 299.974 56.388) (end 301.752 56.388) (width 0.3048) (layer "B.Cu") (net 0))
 (segment (start 297.815 29.337) (end 299.085 28.067) (width 0.3048) (layer "B.Cu") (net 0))
 (segment (start 291.1348 45.847) (end 293.37 45.847) (width 0.3048) (layer "B.Cu") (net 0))
 (segment (start 301.625 46.99) (end 301.625 44.577) (width 0.3048) (layer "B.Cu") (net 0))
 (segment (start 296.545 17.907) (end 296.926 17.907) (width 0.3048) (layer "B.Cu") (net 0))
 (segment (start 294.64 52.832) (end 294.64 29.972) (width 0.3048) (layer "B.Cu") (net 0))
 (segment (start 292.735 42.418) (end 292.735 27.432) (width 0.3048) (layer "B.Cu") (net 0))
 (segment (start 294.005 49.403) (end 294.005 29.337) (width 0.3048) (layer "B.Cu") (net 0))
 (segment (start 294.005 13.462) (end 297.18 13.462) (width 0.3048) (layer "B.Cu") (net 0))
 (segment (start 292.735 19.812) (end 295.91 16.637) (width 0.3048) (layer "B.Cu") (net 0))
 (segment (start 292.735 21.336) (end 292.735 19.812) (width 0.3048) (layer "B.Cu") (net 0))
 (segment (start 294.005 16.002) (end 294.005 13.462) (width 0.3048) (layer "B.Cu") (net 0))
 (segment (start 291.084 56.388) (end 295.275 56.388) (width 0.3048) (layer "B.Cu") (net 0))
 (segment (start 299.339 66.929) (end 301.752 66.929) (width 0.3048) (layer "B.Cu") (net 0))
 (segment (start 297.434 43.307) (end 298.704 44.577) (width 0.3048) (layer "B.Cu") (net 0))
 (segment (start 292.735 27.432) (end 294.64 25.527) (width 0.3048) (layer "B.Cu") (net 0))
 (segment (start 293.37 28.575) (end 295.148 26.797) (width 0.3048) (layer "B.Cu") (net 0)))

